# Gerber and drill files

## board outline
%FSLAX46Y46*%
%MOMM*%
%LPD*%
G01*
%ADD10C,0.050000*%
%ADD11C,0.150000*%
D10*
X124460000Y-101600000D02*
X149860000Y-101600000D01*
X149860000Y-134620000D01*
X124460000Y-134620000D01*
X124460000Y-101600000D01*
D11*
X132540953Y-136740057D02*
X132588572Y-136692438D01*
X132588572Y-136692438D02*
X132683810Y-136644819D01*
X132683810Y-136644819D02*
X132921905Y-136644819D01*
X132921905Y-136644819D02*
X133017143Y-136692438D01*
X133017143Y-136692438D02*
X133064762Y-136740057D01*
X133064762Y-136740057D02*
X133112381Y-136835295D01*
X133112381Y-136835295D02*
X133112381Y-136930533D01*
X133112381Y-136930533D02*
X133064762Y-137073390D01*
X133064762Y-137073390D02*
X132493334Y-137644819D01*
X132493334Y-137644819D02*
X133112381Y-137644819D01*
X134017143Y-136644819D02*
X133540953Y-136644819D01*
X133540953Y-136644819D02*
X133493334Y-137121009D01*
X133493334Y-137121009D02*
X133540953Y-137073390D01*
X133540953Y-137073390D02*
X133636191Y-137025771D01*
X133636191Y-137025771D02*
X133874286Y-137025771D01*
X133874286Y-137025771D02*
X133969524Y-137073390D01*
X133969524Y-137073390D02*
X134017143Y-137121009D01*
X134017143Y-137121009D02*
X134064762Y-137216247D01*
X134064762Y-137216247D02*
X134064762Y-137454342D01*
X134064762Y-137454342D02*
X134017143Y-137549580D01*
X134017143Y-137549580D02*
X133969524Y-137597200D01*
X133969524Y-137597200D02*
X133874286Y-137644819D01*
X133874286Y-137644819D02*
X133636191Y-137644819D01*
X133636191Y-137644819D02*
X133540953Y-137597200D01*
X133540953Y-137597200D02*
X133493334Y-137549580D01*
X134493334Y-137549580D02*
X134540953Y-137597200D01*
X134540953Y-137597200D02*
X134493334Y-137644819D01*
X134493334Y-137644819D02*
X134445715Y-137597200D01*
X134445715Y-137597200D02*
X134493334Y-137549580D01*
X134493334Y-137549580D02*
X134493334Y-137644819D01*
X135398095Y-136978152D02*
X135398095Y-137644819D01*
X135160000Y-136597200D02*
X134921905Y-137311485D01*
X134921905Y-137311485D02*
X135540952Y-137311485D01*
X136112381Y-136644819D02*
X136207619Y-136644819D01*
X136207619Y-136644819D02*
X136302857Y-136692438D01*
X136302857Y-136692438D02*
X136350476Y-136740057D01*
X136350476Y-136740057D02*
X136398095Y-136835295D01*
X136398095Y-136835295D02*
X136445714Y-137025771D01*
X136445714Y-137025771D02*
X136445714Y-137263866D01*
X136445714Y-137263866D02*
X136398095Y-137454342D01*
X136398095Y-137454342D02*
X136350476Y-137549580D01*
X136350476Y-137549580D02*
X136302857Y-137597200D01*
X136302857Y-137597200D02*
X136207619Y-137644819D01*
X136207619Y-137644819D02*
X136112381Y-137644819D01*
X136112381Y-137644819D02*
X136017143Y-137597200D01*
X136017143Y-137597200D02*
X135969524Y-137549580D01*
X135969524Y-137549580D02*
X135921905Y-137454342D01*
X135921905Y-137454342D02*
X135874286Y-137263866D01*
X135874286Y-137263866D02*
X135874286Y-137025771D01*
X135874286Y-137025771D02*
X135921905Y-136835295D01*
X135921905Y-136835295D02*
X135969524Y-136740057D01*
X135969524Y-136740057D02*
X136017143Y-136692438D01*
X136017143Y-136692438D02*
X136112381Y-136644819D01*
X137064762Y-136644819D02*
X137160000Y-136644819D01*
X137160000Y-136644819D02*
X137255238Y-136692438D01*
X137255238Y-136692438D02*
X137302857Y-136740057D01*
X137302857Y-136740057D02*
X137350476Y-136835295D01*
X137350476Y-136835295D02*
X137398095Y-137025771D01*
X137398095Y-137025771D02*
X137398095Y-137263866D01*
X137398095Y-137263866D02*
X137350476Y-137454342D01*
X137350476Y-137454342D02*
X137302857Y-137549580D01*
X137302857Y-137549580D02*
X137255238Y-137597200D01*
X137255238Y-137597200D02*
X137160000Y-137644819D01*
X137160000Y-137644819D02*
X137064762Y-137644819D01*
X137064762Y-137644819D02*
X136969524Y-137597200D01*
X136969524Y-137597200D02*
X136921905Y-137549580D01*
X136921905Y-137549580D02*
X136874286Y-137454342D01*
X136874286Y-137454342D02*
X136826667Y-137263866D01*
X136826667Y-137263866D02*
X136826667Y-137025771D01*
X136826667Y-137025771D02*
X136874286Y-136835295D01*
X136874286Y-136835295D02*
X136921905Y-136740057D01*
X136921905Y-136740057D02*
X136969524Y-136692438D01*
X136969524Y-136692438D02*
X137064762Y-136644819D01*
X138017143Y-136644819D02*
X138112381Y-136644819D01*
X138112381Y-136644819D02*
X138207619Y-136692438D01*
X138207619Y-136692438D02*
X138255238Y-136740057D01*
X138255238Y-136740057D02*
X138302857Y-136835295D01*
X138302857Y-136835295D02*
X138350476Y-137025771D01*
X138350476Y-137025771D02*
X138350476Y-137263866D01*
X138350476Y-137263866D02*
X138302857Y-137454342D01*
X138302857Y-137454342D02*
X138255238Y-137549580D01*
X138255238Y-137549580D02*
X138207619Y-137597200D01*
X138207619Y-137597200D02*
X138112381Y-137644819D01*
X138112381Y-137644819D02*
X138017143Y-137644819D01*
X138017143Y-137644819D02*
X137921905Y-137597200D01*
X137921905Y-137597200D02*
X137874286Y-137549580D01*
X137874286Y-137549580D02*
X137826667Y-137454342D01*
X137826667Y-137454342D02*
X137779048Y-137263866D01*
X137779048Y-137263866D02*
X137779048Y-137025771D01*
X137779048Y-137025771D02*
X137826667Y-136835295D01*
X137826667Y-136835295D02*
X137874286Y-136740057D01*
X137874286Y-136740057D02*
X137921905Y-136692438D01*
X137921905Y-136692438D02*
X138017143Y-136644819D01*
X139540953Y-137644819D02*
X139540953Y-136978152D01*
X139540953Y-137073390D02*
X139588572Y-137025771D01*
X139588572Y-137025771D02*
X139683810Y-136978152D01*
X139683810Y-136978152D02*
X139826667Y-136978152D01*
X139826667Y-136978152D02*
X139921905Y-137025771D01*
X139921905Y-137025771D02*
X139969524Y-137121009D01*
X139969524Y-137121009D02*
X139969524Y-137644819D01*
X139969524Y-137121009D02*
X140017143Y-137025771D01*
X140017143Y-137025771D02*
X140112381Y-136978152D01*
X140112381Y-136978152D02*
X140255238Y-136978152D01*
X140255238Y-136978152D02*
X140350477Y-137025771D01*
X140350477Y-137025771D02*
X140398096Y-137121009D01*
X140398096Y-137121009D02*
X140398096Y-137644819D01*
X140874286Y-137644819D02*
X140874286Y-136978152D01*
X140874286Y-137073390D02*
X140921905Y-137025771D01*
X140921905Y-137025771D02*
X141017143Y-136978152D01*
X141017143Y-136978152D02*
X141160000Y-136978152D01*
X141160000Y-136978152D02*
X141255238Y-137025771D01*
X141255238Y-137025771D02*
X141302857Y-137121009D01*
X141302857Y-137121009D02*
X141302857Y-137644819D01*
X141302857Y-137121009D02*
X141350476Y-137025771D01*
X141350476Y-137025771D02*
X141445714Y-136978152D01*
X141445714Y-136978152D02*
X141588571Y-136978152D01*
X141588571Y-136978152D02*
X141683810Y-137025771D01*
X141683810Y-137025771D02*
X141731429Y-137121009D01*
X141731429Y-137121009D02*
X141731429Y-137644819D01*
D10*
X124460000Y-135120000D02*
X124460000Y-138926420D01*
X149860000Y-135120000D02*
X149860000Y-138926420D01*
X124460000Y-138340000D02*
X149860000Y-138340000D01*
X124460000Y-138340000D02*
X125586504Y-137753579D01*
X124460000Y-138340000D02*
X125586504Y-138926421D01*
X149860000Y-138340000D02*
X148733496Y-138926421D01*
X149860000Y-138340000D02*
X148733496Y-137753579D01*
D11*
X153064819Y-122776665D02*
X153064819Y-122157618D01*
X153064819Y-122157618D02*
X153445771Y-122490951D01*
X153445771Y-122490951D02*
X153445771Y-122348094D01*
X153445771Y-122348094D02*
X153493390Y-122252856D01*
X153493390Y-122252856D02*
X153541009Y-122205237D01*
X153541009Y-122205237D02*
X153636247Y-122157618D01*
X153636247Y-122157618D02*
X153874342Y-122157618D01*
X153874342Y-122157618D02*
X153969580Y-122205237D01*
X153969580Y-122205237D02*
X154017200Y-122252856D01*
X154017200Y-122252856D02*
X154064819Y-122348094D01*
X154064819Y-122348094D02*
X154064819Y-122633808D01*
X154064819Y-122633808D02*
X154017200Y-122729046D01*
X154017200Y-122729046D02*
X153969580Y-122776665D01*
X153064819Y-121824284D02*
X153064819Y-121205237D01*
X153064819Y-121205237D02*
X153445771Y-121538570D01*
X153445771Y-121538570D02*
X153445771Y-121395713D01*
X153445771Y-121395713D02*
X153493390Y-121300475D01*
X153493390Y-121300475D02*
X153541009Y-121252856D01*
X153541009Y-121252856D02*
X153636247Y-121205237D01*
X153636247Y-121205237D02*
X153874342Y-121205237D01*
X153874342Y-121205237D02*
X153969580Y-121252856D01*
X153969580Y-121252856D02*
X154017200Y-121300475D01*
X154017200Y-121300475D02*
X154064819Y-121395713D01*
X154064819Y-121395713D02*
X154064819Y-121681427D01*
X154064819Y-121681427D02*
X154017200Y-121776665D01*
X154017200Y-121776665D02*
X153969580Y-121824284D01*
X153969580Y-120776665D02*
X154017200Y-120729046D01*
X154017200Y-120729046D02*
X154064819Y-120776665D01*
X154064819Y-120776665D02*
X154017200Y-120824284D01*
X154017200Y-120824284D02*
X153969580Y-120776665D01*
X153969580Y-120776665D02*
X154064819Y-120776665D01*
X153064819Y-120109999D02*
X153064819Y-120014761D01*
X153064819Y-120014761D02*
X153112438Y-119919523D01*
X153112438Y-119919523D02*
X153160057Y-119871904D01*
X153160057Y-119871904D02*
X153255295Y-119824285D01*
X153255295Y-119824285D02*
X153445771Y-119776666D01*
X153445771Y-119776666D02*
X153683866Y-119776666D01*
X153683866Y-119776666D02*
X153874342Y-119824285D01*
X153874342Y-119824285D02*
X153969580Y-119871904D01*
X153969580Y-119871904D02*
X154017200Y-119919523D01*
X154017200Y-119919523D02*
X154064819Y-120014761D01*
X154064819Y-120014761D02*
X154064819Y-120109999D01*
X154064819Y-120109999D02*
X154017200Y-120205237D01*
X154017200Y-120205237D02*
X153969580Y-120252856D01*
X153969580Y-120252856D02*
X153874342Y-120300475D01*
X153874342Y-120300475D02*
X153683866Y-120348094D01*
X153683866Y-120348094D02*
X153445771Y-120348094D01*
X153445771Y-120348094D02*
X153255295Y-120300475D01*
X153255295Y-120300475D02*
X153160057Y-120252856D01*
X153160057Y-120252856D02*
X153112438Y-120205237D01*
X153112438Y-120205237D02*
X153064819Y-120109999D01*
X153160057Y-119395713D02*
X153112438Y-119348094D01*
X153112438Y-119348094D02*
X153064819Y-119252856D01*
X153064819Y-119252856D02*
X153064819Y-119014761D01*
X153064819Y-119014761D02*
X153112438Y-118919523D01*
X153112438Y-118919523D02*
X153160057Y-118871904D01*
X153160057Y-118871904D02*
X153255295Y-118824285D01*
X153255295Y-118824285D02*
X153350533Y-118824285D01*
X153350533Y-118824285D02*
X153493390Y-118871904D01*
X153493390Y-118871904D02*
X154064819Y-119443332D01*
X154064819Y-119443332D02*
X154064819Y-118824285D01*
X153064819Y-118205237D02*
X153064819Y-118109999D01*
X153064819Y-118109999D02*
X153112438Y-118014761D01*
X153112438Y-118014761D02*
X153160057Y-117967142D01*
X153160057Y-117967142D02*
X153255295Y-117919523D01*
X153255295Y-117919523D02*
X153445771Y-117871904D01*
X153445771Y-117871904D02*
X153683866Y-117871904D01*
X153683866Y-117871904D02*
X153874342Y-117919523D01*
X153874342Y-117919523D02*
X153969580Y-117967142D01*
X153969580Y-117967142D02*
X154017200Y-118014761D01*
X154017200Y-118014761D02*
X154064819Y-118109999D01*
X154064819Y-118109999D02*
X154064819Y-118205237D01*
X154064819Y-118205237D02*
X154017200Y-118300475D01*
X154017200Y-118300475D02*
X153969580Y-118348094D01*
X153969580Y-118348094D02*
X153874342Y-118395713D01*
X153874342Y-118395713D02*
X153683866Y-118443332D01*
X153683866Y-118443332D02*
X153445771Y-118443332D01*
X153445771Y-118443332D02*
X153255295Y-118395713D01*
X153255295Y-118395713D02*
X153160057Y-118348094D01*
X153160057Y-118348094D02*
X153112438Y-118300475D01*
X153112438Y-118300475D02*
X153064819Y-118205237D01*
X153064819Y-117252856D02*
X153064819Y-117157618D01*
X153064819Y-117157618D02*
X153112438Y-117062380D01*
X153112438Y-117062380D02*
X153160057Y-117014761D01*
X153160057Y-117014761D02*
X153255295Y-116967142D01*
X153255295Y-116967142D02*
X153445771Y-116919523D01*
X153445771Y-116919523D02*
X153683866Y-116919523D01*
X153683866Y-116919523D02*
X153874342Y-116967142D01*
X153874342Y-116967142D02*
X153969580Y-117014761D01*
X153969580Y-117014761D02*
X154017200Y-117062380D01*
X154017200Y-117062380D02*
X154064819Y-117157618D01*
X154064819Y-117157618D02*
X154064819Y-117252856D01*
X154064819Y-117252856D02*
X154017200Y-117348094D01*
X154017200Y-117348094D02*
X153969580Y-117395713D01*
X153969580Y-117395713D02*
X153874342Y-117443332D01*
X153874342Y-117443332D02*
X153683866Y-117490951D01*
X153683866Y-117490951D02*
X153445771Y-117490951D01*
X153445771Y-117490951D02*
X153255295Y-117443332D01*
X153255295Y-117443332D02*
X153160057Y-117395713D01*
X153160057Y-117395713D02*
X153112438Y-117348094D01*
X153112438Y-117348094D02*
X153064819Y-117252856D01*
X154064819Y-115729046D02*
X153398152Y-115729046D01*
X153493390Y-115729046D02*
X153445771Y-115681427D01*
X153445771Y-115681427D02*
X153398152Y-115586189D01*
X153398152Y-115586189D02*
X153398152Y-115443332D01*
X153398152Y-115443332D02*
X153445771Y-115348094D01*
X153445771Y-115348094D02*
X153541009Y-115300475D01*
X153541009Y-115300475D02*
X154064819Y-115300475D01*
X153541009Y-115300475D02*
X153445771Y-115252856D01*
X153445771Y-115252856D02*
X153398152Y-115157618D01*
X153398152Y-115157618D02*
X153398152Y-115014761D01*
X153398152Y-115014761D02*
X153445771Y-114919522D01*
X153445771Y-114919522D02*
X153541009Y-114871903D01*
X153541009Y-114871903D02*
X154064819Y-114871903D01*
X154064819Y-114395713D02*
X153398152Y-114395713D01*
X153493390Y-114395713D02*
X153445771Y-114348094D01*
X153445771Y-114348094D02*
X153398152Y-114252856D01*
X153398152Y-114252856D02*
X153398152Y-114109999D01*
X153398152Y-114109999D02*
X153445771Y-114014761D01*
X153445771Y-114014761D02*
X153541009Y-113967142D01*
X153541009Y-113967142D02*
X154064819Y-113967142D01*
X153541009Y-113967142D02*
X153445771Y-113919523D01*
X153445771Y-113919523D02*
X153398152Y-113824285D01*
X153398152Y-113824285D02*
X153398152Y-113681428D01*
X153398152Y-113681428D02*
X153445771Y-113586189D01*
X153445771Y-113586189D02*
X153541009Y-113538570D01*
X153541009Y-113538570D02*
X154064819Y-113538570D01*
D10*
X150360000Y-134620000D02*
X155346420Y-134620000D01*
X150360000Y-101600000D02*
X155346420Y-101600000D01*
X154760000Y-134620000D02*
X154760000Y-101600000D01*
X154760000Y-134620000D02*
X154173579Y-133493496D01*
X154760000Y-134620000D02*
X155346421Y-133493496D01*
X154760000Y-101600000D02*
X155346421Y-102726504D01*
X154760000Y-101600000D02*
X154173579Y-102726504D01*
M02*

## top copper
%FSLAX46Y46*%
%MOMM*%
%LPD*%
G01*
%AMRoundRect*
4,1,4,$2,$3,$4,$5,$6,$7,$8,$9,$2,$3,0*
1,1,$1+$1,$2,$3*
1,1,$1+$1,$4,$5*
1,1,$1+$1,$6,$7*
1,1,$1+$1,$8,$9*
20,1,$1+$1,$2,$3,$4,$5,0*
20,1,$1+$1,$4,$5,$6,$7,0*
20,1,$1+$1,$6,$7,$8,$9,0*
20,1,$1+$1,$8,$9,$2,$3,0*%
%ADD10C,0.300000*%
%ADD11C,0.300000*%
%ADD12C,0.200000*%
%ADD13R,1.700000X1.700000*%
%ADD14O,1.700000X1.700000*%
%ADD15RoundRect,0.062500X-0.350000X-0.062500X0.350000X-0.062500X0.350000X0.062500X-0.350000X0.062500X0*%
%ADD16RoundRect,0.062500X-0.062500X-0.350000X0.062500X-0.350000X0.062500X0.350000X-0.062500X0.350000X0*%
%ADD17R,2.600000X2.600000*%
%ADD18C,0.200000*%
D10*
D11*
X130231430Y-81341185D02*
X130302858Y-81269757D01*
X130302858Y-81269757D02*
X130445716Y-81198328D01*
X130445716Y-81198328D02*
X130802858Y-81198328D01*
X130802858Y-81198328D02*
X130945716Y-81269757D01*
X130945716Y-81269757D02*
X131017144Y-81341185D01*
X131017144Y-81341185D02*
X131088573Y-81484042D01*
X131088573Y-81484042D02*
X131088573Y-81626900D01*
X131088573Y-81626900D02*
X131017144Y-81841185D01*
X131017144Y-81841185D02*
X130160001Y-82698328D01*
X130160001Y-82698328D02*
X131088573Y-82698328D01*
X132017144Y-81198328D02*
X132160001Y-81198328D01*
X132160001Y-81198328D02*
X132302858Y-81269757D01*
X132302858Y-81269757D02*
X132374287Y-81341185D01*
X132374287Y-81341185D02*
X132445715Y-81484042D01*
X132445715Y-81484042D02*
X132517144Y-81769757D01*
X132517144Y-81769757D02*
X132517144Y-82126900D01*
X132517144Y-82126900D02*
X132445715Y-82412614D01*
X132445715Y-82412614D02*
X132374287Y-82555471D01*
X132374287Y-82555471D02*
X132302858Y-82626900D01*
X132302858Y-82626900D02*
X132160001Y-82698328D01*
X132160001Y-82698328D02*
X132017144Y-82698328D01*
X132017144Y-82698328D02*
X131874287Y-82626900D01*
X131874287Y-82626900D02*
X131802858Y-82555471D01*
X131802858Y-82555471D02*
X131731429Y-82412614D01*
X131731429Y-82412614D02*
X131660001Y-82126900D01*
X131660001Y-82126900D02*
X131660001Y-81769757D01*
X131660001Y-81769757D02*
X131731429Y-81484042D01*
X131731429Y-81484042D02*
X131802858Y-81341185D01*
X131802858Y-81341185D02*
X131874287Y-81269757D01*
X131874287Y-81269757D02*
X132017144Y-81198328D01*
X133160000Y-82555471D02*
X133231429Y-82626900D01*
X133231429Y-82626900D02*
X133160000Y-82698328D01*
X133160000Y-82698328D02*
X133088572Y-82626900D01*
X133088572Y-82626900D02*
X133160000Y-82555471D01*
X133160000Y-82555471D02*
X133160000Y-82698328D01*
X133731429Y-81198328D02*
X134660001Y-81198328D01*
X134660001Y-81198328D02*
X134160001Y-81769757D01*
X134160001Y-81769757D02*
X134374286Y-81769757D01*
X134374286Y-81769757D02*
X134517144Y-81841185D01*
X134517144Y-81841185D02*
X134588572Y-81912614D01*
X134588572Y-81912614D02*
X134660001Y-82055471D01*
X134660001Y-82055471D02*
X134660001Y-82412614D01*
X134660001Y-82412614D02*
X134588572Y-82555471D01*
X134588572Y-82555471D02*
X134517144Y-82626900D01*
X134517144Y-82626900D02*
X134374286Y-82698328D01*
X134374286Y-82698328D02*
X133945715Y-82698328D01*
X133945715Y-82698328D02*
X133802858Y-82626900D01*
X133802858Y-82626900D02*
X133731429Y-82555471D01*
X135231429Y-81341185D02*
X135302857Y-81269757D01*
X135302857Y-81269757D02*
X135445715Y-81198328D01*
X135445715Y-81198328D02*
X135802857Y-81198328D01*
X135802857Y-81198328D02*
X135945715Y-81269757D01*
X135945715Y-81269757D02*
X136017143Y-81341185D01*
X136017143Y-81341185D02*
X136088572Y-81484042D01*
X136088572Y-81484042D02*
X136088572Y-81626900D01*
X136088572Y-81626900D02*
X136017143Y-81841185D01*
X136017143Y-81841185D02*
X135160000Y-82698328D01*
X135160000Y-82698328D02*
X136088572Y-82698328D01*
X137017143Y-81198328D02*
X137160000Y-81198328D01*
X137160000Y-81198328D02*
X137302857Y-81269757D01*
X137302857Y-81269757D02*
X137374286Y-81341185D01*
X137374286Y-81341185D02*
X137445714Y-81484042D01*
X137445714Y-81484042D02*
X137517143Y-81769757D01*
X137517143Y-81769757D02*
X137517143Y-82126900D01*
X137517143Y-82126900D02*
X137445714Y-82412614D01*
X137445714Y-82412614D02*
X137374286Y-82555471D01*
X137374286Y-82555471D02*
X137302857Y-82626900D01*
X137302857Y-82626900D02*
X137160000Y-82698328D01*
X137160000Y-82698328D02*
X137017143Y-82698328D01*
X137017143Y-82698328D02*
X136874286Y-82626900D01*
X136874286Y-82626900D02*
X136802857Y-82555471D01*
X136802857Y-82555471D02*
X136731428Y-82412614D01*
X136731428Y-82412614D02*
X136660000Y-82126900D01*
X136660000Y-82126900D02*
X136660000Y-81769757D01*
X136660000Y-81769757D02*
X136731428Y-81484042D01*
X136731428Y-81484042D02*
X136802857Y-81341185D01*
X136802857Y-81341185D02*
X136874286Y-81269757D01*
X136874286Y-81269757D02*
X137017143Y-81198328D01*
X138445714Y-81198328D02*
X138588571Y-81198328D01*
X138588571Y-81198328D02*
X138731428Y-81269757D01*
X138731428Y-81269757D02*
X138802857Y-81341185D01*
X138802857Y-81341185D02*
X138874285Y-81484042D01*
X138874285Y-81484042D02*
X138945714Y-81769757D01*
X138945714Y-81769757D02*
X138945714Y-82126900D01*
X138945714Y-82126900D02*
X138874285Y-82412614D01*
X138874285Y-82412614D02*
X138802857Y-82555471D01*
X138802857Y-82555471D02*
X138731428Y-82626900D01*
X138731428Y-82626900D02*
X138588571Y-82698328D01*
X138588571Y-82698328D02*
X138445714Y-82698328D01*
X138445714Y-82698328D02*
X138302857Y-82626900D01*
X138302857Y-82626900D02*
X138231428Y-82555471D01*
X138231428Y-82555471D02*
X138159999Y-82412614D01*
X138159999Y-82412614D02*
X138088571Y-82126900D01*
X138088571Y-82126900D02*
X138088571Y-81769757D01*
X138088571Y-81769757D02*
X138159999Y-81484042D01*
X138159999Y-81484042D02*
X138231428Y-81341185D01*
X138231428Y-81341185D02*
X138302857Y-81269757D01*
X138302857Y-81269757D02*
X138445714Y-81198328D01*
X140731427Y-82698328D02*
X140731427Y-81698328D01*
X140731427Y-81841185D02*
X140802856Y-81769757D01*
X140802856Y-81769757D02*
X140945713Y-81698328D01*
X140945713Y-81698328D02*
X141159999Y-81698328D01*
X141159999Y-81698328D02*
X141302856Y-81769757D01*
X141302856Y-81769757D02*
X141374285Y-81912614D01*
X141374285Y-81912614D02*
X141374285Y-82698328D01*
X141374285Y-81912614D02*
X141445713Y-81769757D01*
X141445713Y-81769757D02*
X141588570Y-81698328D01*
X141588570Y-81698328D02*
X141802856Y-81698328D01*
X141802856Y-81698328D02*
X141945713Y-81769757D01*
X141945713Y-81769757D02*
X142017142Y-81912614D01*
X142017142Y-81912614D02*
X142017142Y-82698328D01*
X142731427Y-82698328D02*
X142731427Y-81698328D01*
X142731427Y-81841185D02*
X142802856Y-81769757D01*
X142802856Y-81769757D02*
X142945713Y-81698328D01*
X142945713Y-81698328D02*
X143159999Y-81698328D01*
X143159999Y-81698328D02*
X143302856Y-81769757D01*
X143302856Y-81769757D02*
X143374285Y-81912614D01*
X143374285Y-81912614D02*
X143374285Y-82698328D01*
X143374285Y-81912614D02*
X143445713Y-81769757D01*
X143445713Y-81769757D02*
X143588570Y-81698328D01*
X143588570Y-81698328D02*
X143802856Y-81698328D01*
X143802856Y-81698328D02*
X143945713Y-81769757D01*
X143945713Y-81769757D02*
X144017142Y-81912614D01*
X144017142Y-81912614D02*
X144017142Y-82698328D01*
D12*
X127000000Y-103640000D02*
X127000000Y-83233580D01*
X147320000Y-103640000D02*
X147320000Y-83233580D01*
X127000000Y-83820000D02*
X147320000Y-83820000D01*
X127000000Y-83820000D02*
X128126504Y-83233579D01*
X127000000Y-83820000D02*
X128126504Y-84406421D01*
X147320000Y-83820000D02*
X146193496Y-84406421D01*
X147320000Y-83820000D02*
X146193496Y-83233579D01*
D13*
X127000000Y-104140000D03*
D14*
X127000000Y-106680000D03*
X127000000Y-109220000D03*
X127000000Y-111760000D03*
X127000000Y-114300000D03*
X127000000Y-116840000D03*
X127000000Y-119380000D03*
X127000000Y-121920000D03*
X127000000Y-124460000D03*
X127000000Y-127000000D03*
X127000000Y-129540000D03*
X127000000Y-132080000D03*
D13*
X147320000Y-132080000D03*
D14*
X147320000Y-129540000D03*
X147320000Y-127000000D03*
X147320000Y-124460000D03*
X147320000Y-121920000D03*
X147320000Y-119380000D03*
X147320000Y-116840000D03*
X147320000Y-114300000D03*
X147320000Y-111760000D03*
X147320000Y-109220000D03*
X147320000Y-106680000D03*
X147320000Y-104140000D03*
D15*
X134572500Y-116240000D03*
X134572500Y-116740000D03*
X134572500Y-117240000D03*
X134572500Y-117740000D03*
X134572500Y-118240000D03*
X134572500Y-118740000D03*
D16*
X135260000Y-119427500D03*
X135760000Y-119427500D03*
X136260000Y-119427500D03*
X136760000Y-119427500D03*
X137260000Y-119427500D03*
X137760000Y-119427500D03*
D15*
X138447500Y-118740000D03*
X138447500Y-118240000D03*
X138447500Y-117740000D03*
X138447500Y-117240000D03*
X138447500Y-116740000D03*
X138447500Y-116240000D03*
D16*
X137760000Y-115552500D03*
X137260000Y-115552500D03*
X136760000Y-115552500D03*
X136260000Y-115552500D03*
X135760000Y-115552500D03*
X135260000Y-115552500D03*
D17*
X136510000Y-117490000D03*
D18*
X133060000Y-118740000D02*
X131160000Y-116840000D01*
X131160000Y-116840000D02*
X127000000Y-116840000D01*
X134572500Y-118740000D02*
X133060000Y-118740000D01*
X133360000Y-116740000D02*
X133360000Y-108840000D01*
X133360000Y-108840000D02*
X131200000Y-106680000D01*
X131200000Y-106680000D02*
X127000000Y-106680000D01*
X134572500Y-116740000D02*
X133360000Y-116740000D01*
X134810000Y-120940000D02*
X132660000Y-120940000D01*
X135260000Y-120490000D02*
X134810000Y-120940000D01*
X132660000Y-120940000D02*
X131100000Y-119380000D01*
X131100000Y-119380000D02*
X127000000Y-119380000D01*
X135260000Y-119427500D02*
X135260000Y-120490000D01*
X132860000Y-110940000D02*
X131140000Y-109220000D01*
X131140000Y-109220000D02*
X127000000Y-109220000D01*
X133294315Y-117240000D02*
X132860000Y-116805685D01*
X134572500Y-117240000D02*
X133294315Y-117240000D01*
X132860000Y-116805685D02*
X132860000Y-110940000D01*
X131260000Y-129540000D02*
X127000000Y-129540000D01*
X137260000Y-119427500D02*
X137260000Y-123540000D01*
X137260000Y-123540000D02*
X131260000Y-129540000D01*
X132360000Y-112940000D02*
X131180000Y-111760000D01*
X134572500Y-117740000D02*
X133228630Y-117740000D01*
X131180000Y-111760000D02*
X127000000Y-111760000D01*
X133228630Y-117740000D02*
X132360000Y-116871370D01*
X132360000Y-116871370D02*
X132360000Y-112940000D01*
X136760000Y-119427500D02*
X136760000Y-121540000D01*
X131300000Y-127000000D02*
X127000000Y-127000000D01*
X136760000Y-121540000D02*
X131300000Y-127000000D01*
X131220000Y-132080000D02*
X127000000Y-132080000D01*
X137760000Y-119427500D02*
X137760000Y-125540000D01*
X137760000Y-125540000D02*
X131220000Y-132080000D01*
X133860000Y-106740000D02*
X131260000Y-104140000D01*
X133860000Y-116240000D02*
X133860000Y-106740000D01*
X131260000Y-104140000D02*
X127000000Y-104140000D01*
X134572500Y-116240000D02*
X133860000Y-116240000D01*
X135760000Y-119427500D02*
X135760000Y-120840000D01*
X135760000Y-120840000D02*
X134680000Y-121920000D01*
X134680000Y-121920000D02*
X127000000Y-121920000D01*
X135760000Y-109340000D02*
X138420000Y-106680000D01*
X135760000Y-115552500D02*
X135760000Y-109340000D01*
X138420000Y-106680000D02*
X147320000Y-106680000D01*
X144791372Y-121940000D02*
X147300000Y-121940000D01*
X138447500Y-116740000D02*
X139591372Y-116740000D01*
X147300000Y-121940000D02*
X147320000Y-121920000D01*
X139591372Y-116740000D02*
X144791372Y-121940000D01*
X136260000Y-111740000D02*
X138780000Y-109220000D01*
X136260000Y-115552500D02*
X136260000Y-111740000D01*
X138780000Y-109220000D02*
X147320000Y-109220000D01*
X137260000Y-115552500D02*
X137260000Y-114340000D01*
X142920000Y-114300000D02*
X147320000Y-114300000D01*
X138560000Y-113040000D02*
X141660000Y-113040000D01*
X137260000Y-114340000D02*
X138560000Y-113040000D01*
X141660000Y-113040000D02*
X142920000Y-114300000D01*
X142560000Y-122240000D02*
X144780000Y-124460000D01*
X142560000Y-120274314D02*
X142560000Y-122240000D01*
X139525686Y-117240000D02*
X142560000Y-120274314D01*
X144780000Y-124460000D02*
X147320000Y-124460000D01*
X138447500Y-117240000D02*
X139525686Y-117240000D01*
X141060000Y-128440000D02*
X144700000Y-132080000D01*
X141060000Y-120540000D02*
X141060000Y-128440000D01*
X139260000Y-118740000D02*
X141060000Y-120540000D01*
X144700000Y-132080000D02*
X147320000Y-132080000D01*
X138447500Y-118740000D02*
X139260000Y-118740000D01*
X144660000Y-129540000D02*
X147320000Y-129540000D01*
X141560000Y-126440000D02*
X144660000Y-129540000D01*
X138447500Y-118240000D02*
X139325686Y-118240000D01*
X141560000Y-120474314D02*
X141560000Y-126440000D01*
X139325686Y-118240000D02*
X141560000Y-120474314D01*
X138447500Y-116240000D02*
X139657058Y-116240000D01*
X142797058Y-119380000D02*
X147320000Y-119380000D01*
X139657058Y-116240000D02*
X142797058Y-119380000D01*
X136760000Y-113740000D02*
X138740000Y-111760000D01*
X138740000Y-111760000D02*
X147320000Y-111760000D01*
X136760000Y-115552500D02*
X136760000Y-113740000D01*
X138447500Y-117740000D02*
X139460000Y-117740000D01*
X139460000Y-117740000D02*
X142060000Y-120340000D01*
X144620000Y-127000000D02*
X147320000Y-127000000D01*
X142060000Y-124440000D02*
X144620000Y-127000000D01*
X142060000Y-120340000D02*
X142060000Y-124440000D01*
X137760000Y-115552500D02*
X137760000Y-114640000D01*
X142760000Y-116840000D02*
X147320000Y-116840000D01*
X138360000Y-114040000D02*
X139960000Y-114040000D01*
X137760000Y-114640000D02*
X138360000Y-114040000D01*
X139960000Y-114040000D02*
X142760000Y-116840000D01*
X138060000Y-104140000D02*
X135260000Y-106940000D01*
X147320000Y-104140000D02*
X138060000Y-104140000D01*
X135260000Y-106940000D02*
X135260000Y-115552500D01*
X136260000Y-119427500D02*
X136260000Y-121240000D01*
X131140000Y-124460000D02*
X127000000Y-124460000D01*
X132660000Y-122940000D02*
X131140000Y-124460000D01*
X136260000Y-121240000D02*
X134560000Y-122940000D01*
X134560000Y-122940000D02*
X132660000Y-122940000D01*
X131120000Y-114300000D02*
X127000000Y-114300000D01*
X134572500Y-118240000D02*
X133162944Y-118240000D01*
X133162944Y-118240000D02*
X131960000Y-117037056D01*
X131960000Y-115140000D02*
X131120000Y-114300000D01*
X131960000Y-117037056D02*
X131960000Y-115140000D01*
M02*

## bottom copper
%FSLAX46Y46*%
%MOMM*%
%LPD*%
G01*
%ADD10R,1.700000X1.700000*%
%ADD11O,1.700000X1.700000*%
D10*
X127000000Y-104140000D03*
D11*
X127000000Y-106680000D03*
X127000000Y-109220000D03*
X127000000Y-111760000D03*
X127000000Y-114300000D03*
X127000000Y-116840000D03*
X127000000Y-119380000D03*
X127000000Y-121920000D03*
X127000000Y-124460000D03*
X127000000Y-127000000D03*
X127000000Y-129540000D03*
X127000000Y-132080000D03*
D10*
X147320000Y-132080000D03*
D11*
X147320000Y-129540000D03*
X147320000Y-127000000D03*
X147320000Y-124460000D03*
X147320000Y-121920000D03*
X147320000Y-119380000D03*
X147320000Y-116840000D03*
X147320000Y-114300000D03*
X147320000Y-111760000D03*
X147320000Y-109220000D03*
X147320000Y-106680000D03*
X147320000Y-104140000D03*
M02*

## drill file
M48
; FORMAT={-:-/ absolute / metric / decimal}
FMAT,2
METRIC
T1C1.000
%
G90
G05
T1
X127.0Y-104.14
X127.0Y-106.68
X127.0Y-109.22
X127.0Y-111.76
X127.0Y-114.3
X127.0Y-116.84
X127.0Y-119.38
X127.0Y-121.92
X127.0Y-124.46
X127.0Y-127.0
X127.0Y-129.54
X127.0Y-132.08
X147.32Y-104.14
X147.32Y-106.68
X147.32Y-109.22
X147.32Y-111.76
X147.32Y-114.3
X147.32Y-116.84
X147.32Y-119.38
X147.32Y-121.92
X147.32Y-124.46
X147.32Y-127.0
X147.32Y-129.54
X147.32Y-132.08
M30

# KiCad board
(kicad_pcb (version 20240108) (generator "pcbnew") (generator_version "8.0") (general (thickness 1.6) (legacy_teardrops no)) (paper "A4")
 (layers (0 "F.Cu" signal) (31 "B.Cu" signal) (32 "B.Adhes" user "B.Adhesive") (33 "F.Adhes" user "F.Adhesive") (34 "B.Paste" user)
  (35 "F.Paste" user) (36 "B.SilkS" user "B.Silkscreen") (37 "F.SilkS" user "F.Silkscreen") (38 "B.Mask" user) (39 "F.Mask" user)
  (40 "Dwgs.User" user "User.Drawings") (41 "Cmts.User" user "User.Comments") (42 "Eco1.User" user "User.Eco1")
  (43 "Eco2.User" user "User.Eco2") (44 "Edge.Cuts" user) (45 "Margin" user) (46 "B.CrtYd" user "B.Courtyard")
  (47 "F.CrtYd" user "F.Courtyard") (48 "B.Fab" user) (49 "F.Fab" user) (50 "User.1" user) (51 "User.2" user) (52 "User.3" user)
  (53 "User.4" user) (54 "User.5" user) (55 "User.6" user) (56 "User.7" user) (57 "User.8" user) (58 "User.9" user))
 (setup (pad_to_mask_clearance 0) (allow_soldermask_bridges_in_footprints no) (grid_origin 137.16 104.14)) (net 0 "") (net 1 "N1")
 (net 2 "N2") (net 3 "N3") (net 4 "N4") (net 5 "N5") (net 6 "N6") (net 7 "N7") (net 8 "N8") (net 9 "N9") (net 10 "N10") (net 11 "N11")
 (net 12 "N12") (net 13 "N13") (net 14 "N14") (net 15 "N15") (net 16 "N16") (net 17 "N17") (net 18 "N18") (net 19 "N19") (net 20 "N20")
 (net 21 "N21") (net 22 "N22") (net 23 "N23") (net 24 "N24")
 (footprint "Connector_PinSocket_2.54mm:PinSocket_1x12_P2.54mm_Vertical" (layer "F.Cu") (at 127 104.14)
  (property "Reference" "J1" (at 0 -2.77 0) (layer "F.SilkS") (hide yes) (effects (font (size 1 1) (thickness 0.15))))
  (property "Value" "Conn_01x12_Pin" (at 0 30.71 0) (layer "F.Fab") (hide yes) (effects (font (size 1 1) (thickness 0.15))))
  (pad "1" thru_hole rect (at 0 0) (size 1.7 1.7) (drill 1) (layers "*.Cu" "*.Mask") (remove_unused_layers no) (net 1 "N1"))
  (pad "2" thru_hole oval (at 0 2.54) (size 1.7 1.7) (drill 1) (layers "*.Cu" "*.Mask") (remove_unused_layers no) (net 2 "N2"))
  (pad "3" thru_hole oval (at 0 5.08) (size 1.7 1.7) (drill 1) (layers "*.Cu" "*.Mask") (remove_unused_layers no) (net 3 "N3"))
  (pad "4" thru_hole oval (at 0 7.62) (size 1.7 1.7) (drill 1) (layers "*.Cu" "*.Mask") (remove_unused_layers no) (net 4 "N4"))
  (pad "5" thru_hole oval (at 0 10.16) (size 1.7 1.7) (drill 1) (layers "*.Cu" "*.Mask") (remove_unused_layers no) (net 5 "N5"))
  (pad "6" thru_hole oval (at 0 12.7) (size 1.7 1.7) (drill 1) (layers "*.Cu" "*.Mask") (remove_unused_layers no) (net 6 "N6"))
  (pad "7" thru_hole oval (at 0 15.24) (size 1.7 1.7) (drill 1) (layers "*.Cu" "*.Mask") (remove_unused_layers no) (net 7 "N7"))
  (pad "8" thru_hole oval (at 0 17.78) (size 1.7 1.7) (drill 1) (layers "*.Cu" "*.Mask") (remove_unused_layers no) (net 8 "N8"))
  (pad "9" thru_hole oval (at 0 20.32) (size 1.7 1.7) (drill 1) (layers "*.Cu" "*.Mask") (remove_unused_layers no) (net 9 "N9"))
  (pad "10" thru_hole oval (at 0 22.86) (size 1.7 1.7) (drill 1) (layers "*.Cu" "*.Mask") (remove_unused_layers no) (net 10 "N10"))
  (pad "11" thru_hole oval (at 0 25.4) (size 1.7 1.7) (drill 1) (layers "*.Cu" "*.Mask") (remove_unused_layers no) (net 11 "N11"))
  (pad "12" thru_hole oval (at 0 27.94) (size 1.7 1.7) (drill 1) (layers "*.Cu" "*.Mask") (remove_unused_layers no) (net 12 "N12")))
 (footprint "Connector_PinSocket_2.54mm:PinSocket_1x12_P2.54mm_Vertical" (layer "F.Cu") (at 147.32 132.08 180)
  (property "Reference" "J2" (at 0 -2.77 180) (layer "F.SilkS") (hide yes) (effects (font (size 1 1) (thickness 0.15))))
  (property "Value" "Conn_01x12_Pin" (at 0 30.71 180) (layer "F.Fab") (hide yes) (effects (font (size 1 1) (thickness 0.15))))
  (pad "1" thru_hole rect (at 0 0 180) (size 1.7 1.7) (drill 1) (layers "*.Cu" "*.Mask") (remove_unused_layers no) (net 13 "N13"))
  (pad "2" thru_hole oval (at 0 2.54 180) (size 1.7 1.7) (drill 1) (layers "*.Cu" "*.Mask") (remove_unused_layers no) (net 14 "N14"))
  (pad "3" thru_hole oval (at 0 5.08 180) (size 1.7 1.7) (drill 1) (layers "*.Cu" "*.Mask") (remove_unused_layers no) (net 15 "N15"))
  (pad "4" thru_hole oval (at 0 7.62 180) (size 1.7 1.7) (drill 1) (layers "*.Cu" "*.Mask") (remove_unused_layers no) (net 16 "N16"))
  (pad "5" thru_hole oval (at 0 10.16 180) (size 1.7 1.7) (drill 1) (layers "*.Cu" "*.Mask") (remove_unused_layers no) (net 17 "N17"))
  (pad "6" thru_hole oval (at 0 12.7 180) (size 1.7 1.7) (drill 1) (layers "*.Cu" "*.Mask") (remove_unused_layers no) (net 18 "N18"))
  (pad "7" thru_hole oval (at 0 15.24 180) (size 1.7 1.7) (drill 1) (layers "*.Cu" "*.Mask") (remove_unused_layers no) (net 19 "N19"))
  (pad "8" thru_hole oval (at 0 17.78 180) (size 1.7 1.7) (drill 1) (layers "*.Cu" "*.Mask") (remove_unused_layers no) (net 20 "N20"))
  (pad "9" thru_hole oval (at 0 20.32 180) (size 1.7 1.7) (drill 1) (layers "*.Cu" "*.Mask") (remove_unused_layers no) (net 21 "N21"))
  (pad "10" thru_hole oval (at 0 22.86 180) (size 1.7 1.7) (drill 1) (layers "*.Cu" "*.Mask") (remove_unused_layers no) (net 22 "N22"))
  (pad "11" thru_hole oval (at 0 25.4 180) (size 1.7 1.7) (drill 1) (layers "*.Cu" "*.Mask") (remove_unused_layers no) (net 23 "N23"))
  (pad "12" thru_hole oval (at 0 27.94 180) (size 1.7 1.7) (drill 1) (layers "*.Cu" "*.Mask") (remove_unused_layers no) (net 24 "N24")))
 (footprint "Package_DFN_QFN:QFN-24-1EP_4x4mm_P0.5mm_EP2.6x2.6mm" (layer "F.Cu") (at 136.51 117.49)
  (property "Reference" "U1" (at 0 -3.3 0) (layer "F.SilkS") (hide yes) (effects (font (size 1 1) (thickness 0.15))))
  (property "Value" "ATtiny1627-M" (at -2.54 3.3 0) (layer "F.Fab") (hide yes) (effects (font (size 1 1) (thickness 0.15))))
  (pad "" smd roundrect (at -0.65 -0.65) (size 1.05 1.05) (layers "F.Paste") (roundrect_rratio 0.238095))
  (pad "" smd roundrect (at -0.65 0.65) (size 1.05 1.05) (layers "F.Paste") (roundrect_rratio 0.238095))
  (pad "" smd roundrect (at 0.65 -0.65) (size 1.05 1.05) (layers "F.Paste") (roundrect_rratio 0.238095))
  (pad "" smd roundrect (at 0.65 0.65) (size 1.05 1.05) (layers "F.Paste") (roundrect_rratio 0.238095))
  (pad "1" smd roundrect (at -1.9375 -1.25) (size 0.825 0.25) (layers "F.Cu" "F.Paste" "F.Mask") (roundrect_rratio 0.25) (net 1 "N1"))
  (pad "2" smd roundrect (at -1.9375 -0.75) (size 0.825 0.25) (layers "F.Cu" "F.Paste" "F.Mask") (roundrect_rratio 0.25) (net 2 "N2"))
  (pad "3" smd roundrect (at -1.9375 -0.25) (size 0.825 0.25) (layers "F.Cu" "F.Paste" "F.Mask") (roundrect_rratio 0.25) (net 3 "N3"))
  (pad "4" smd roundrect (at -1.9375 0.25) (size 0.825 0.25) (layers "F.Cu" "F.Paste" "F.Mask") (roundrect_rratio 0.25) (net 4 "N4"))
  (pad "5" smd roundrect (at -1.9375 0.75) (size 0.825 0.25) (layers "F.Cu" "F.Paste" "F.Mask") (roundrect_rratio 0.25) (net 5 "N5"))
  (pad "6" smd roundrect (at -1.9375 1.25) (size 0.825 0.25) (layers "F.Cu" "F.Paste" "F.Mask") (roundrect_rratio 0.25) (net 6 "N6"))
  (pad "7" smd roundrect (at -1.25 1.9375) (size 0.25 0.825) (layers "F.Cu" "F.Paste" "F.Mask") (roundrect_rratio 0.25) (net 7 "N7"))
  (pad "8" smd roundrect (at -0.75 1.9375) (size 0.25 0.825) (layers "F.Cu" "F.Paste" "F.Mask") (roundrect_rratio 0.25) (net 8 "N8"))
  (pad "9" smd roundrect (at -0.25 1.9375) (size 0.25 0.825) (layers "F.Cu" "F.Paste" "F.Mask") (roundrect_rratio 0.25) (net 9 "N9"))
  (pad "10" smd roundrect (at 0.25 1.9375) (size 0.25 0.825) (layers "F.Cu" "F.Paste" "F.Mask") (roundrect_rratio 0.25) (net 10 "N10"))
  (pad "11" smd roundrect (at 0.75 1.9375) (size 0.25 0.825) (layers "F.Cu" "F.Paste" "F.Mask") (roundrect_rratio 0.25) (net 11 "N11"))
  (pad "12" smd roundrect (at 1.25 1.9375) (size 0.25 0.825) (layers "F.Cu" "F.Paste" "F.Mask") (roundrect_rratio 0.25) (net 12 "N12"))
  (pad "13" smd roundrect (at 1.9375 1.25) (size 0.825 0.25) (layers "F.Cu" "F.Paste" "F.Mask") (roundrect_rratio 0.25) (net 13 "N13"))
  (pad "14" smd roundrect (at 1.9375 0.75) (size 0.825 0.25) (layers "F.Cu" "F.Paste" "F.Mask") (roundrect_rratio 0.25) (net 14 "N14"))
  (pad "15" smd roundrect (at 1.9375 0.25) (size 0.825 0.25) (layers "F.Cu" "F.Paste" "F.Mask") (roundrect_rratio 0.25) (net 15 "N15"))
  (pad "16" smd roundrect (at 1.9375 -0.25) (size 0.825 0.25) (layers "F.Cu" "F.Paste" "F.Mask") (roundrect_rratio 0.25) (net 16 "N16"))
  (pad "17" smd roundrect (at 1.9375 -0.75) (size 0.825 0.25) (layers "F.Cu" "F.Paste" "F.Mask") (roundrect_rratio 0.25) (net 17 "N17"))
  (pad "18" smd roundrect (at 1.9375 -1.25) (size 0.825 0.25) (layers "F.Cu" "F.Paste" "F.Mask") (roundrect_rratio 0.25) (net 18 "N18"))
  (pad "19" smd roundrect (at 1.25 -1.9375) (size 0.25 0.825) (layers "F.Cu" "F.Paste" "F.Mask") (roundrect_rratio 0.25) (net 19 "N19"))
  (pad "20" smd roundrect (at 0.75 -1.9375) (size 0.25 0.825) (layers "F.Cu" "F.Paste" "F.Mask") (roundrect_rratio 0.25) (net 20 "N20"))
  (pad "21" smd roundrect (at 0.25 -1.9375) (size 0.25 0.825) (layers "F.Cu" "F.Paste" "F.Mask") (roundrect_rratio 0.25) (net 21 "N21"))
  (pad "22" smd roundrect (at -0.25 -1.9375) (size 0.25 0.825) (layers "F.Cu" "F.Paste" "F.Mask") (roundrect_rratio 0.25) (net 22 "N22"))
  (pad "23" smd roundrect (at -0.75 -1.9375) (size 0.25 0.825) (layers "F.Cu" "F.Paste" "F.Mask") (roundrect_rratio 0.25) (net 23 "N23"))
  (pad "24" smd roundrect (at -1.25 -1.9375) (size 0.25 0.825) (layers "F.Cu" "F.Paste" "F.Mask") (roundrect_rratio 0.25) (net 24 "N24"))
  (pad "25" smd rect (at 0 0) (size 2.6 2.6) (layers "F.Cu" "F.Mask") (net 3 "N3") (zone_connect 2)))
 (gr_rect (start 124.46 101.6) (end 149.86 134.62) (stroke (width 0.05) (type default)) (fill none) (layer "Edge.Cuts"))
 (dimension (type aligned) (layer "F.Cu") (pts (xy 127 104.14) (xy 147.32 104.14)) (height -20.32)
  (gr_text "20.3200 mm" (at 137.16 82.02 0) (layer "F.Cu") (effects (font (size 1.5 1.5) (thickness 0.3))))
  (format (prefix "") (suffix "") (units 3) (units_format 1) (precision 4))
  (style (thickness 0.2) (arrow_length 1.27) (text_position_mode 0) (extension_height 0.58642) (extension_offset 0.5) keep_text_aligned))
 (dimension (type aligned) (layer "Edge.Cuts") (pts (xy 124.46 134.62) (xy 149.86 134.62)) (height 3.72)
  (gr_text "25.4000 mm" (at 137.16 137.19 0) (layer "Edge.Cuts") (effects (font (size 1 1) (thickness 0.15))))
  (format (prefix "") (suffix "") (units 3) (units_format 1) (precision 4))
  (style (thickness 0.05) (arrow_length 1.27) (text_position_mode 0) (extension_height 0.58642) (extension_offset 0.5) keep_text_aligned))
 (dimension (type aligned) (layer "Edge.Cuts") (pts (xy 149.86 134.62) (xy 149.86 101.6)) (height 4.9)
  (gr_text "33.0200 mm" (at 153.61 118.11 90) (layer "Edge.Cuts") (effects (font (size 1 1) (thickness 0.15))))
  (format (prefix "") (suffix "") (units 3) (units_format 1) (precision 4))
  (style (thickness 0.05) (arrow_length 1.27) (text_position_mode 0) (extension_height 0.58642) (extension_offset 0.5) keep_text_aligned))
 (segment (start 133.06 118.74) (end 131.16 116.84) (width 0.2) (layer "F.Cu") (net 6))
 (segment (start 131.16 116.84) (end 127 116.84) (width 0.2) (layer "F.Cu") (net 6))
 (segment (start 134.5725 118.74) (end 133.06 118.74) (width 0.2) (layer "F.Cu") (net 6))
 (segment (start 133.36 116.74) (end 133.36 108.84) (width 0.2) (layer "F.Cu") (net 2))
 (segment (start 133.36 108.84) (end 131.2 106.68) (width 0.2) (layer "F.Cu") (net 2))
 (segment (start 131.2 106.68) (end 127 106.68) (width 0.2) (layer "F.Cu") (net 2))
 (segment (start 134.5725 116.74) (end 133.36 116.74) (width 0.2) (layer "F.Cu") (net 2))
 (segment (start 134.81 120.94) (end 132.66 120.94) (width 0.2) (layer "F.Cu") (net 7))
 (segment (start 135.26 120.49) (end 134.81 120.94) (width 0.2) (layer "F.Cu") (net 7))
 (segment (start 132.66 120.94) (end 131.1 119.38) (width 0.2) (layer "F.Cu") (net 7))
 (segment (start 131.1 119.38) (end 127 119.38) (width 0.2) (layer "F.Cu") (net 7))
 (segment (start 135.26 119.4275) (end 135.26 120.49) (width 0.2) (layer "F.Cu") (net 7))
 (segment (start 132.86 110.94) (end 131.14 109.22) (width 0.2) (layer "F.Cu") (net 3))
 (segment (start 131.14 109.22) (end 127 109.22) (width 0.2) (layer "F.Cu") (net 3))
 (segment (start 133.294315 117.24) (end 132.86 116.805685) (width 0.2) (layer "F.Cu") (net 3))
 (segment (start 134.5725 117.24) (end 133.294315 117.24) (width 0.2) (layer "F.Cu") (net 3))
 (segment (start 132.86 116.805685) (end 132.86 110.94) (width 0.2) (layer "F.Cu") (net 3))
 (segment (start 131.26 129.54) (end 127 129.54) (width 0.2) (layer "F.Cu") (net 11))
 (segment (start 137.26 119.4275) (end 137.26 123.54) (width 0.2) (layer "F.Cu") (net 11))
 (segment (start 137.26 123.54) (end 131.26 129.54) (width 0.2) (layer "F.Cu") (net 11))
 (segment (start 132.36 112.94) (end 131.18 111.76) (width 0.2) (layer "F.Cu") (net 4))
 (segment (start 134.5725 117.74) (end 133.22863 117.74) (width 0.2) (layer "F.Cu") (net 4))
 (segment (start 131.18 111.76) (end 127 111.76) (width 0.2) (layer "F.Cu") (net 4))
 (segment (start 133.22863 117.74) (end 132.36 116.87137) (width 0.2) (layer "F.Cu") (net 4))
 (segment (start 132.36 116.87137) (end 132.36 112.94) (width 0.2) (layer "F.Cu") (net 4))
 (segment (start 136.76 119.4275) (end 136.76 121.54) (width 0.2) (layer "F.Cu") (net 10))
 (segment (start 131.3 127) (end 127 127) (width 0.2) (layer "F.Cu") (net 10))
 (segment (start 136.76 121.54) (end 131.3 127) (width 0.2) (layer "F.Cu") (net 10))
 (segment (start 131.22 132.08) (end 127 132.08) (width 0.2) (layer "F.Cu") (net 12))
 (segment (start 137.76 119.4275) (end 137.76 125.54) (width 0.2) (layer "F.Cu") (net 12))
 (segment (start 137.76 125.54) (end 131.22 132.08) (width 0.2) (layer "F.Cu") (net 12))
 (segment (start 133.86 106.74) (end 131.26 104.14) (width 0.2) (layer "F.Cu") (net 1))
 (segment (start 133.86 116.24) (end 133.86 106.74) (width 0.2) (layer "F.Cu") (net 1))
 (segment (start 131.26 104.14) (end 127 104.14) (width 0.2) (layer "F.Cu") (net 1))
 (segment (start 134.5725 116.24) (end 133.86 116.24) (width 0.2) (layer "F.Cu") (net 1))
 (segment (start 135.76 119.4275) (end 135.76 120.84) (width 0.2) (layer "F.Cu") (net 8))
 (segment (start 135.76 120.84) (end 134.68 121.92) (width 0.2) (layer "F.Cu") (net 8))
 (segment (start 134.68 121.92) (end 127 121.92) (width 0.2) (layer "F.Cu") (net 8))
 (segment (start 135.76 109.34) (end 138.42 106.68) (width 0.2) (layer "F.Cu") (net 23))
 (segment (start 135.76 115.5525) (end 135.76 109.34) (width 0.2) (layer "F.Cu") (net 23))
 (segment (start 138.42 106.68) (end 147.32 106.68) (width 0.2) (layer "F.Cu") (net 23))
 (segment (start 144.791372 121.94) (end 147.3 121.94) (width 0.2) (layer "F.Cu") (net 17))
 (segment (start 138.4475 116.74) (end 139.591372 116.74) (width 0.2) (layer "F.Cu") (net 17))
 (segment (start 147.3 121.94) (end 147.32 121.92) (width 0.2) (layer "F.Cu") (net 17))
 (segment (start 139.591372 116.74) (end 144.791372 121.94) (width 0.2) (layer "F.Cu") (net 17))
 (segment (start 136.26 111.74) (end 138.78 109.22) (width 0.2) (layer "F.Cu") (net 22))
 (segment (start 136.26 115.5525) (end 136.26 111.74) (width 0.2) (layer "F.Cu") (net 22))
 (segment (start 138.78 109.22) (end 147.32 109.22) (width 0.2) (layer "F.Cu") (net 22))
 (segment (start 137.26 115.5525) (end 137.26 114.34) (width 0.2) (layer "F.Cu") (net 20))
 (segment (start 142.92 114.3) (end 147.32 114.3) (width 0.2) (layer "F.Cu") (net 20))
 (segment (start 138.56 113.04) (end 141.66 113.04) (width 0.2) (layer "F.Cu") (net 20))
 (segment (start 137.26 114.34) (end 138.56 113.04) (width 0.2) (layer "F.Cu") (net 20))
 (segment (start 141.66 113.04) (end 142.92 114.3) (width 0.2) (layer "F.Cu") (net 20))
 (segment (start 142.56 122.24) (end 144.78 124.46) (width 0.2) (layer "F.Cu") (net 16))
 (segment (start 142.56 120.274314) (end 142.56 122.24) (width 0.2) (layer "F.Cu") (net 16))
 (segment (start 139.525686 117.24) (end 142.56 120.274314) (width 0.2) (layer "F.Cu") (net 16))
 (segment (start 144.78 124.46) (end 147.32 124.46) (width 0.2) (layer "F.Cu") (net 16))
 (segment (start 138.4475 117.24) (end 139.525686 117.24) (width 0.2) (layer "F.Cu") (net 16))
 (segment (start 141.06 128.44) (end 144.7 132.08) (width 0.2) (layer "F.Cu") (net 13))
 (segment (start 141.06 120.54) (end 141.06 128.44) (width 0.2) (layer "F.Cu") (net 13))
 (segment (start 139.26 118.74) (end 141.06 120.54) (width 0.2) (layer "F.Cu") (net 13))
 (segment (start 144.7 132.08) (end 147.32 132.08) (width 0.2) (layer "F.Cu") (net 13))
 (segment (start 138.4475 118.74) (end 139.26 118.74) (width 0.2) (layer "F.Cu") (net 13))
 (segment (start 144.66 129.54) (end 147.32 129.54) (width 0.2) (layer "F.Cu") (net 14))
 (segment (start 141.56 126.44) (end 144.66 129.54) (width 0.2) (layer "F.Cu") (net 14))
 (segment (start 138.4475 118.24) (end 139.325686 118.24) (width 0.2) (layer "F.Cu") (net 14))
 (segment (start 141.56 120.474314) (end 141.56 126.44) (width 0.2) (layer "F.Cu") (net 14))
 (segment (start 139.325686 118.24) (end 141.56 120.474314) (width 0.2) (layer "F.Cu") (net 14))
 (segment (start 138.4475 116.24) (end 139.657058 116.24) (width 0.2) (layer "F.Cu") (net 18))
 (segment (start 142.797058 119.38) (end 147.32 119.38) (width 0.2) (layer "F.Cu") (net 18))
 (segment (start 139.657058 116.24) (end 142.797058 119.38) (width 0.2) (layer "F.Cu") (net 18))
 (segment (start 136.76 113.74) (end 138.74 111.76) (width 0.2) (layer "F.Cu") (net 21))
 (segment (start 138.74 111.76) (end 147.32 111.76) (width 0.2) (layer "F.Cu") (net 21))
 (segment (start 136.76 115.5525) (end 136.76 113.74) (width 0.2) (layer "F.Cu") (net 21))
 (segment (start 138.4475 117.74) (end 139.46 117.74) (width 0.2) (layer "F.Cu") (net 15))
 (segment (start 139.46 117.74) (end 142.06 120.34) (width 0.2) (layer "F.Cu") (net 15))
 (segment (start 144.62 127) (end 147.32 127) (width 0.2) (layer "F.Cu") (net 15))
 (segment (start 142.06 124.44) (end 144.62 127) (width 0.2) (layer "F.Cu") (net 15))
 (segment (start 142.06 120.34) (end 142.06 124.44) (width 0.2) (layer "F.Cu") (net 15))
 (segment (start 137.76 115.5525) (end 137.76 114.64) (width 0.2) (layer "F.Cu") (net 19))
 (segment (start 142.76 116.84) (end 147.32 116.84) (width 0.2) (layer "F.Cu") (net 19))
 (segment (start 138.36 114.04) (end 139.96 114.04) (width 0.2) (layer "F.Cu") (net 19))
 (segment (start 137.76 114.64) (end 138.36 114.04) (width 0.2) (layer "F.Cu") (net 19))
 (segment (start 139.96 114.04) (end 142.76 116.84) (width 0.2) (layer "F.Cu") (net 19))
 (segment (start 138.06 104.14) (end 135.26 106.94) (width 0.2) (layer "F.Cu") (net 24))
 (segment (start 147.32 104.14) (end 138.06 104.14) (width 0.2) (layer "F.Cu") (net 24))
 (segment (start 135.26 106.94) (end 135.26 115.5525) (width 0.2) (layer "F.Cu") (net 24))
 (segment (start 136.26 119.4275) (end 136.26 121.24) (width 0.2) (layer "F.Cu") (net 9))
 (segment (start 131.14 124.46) (end 127 124.46) (width 0.2) (layer "F.Cu") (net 9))
 (segment (start 132.66 122.94) (end 131.14 124.46) (width 0.2) (layer "F.Cu") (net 9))
 (segment (start 136.26 121.24) (end 134.56 122.94) (width 0.2) (layer "F.Cu") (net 9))
 (segment (start 134.56 122.94) (end 132.66 122.94) (width 0.2) (layer "F.Cu") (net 9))
 (segment (start 131.12 114.3) (end 127 114.3) (width 0.2) (layer "F.Cu") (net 5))
 (segment (start 134.5725 118.24) (end 133.162944 118.24) (width 0.2) (layer "F.Cu") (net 5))
 (segment (start 133.162944 118.24) (end 131.96 117.037056) (width 0.2) (layer "F.Cu") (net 5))
 (segment (start 131.96 115.14) (end 131.12 114.3) (width 0.2) (layer "F.Cu") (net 5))
 (segment (start 131.96 117.037056) (end 131.96 115.14) (width 0.2) (layer "F.Cu") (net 5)))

